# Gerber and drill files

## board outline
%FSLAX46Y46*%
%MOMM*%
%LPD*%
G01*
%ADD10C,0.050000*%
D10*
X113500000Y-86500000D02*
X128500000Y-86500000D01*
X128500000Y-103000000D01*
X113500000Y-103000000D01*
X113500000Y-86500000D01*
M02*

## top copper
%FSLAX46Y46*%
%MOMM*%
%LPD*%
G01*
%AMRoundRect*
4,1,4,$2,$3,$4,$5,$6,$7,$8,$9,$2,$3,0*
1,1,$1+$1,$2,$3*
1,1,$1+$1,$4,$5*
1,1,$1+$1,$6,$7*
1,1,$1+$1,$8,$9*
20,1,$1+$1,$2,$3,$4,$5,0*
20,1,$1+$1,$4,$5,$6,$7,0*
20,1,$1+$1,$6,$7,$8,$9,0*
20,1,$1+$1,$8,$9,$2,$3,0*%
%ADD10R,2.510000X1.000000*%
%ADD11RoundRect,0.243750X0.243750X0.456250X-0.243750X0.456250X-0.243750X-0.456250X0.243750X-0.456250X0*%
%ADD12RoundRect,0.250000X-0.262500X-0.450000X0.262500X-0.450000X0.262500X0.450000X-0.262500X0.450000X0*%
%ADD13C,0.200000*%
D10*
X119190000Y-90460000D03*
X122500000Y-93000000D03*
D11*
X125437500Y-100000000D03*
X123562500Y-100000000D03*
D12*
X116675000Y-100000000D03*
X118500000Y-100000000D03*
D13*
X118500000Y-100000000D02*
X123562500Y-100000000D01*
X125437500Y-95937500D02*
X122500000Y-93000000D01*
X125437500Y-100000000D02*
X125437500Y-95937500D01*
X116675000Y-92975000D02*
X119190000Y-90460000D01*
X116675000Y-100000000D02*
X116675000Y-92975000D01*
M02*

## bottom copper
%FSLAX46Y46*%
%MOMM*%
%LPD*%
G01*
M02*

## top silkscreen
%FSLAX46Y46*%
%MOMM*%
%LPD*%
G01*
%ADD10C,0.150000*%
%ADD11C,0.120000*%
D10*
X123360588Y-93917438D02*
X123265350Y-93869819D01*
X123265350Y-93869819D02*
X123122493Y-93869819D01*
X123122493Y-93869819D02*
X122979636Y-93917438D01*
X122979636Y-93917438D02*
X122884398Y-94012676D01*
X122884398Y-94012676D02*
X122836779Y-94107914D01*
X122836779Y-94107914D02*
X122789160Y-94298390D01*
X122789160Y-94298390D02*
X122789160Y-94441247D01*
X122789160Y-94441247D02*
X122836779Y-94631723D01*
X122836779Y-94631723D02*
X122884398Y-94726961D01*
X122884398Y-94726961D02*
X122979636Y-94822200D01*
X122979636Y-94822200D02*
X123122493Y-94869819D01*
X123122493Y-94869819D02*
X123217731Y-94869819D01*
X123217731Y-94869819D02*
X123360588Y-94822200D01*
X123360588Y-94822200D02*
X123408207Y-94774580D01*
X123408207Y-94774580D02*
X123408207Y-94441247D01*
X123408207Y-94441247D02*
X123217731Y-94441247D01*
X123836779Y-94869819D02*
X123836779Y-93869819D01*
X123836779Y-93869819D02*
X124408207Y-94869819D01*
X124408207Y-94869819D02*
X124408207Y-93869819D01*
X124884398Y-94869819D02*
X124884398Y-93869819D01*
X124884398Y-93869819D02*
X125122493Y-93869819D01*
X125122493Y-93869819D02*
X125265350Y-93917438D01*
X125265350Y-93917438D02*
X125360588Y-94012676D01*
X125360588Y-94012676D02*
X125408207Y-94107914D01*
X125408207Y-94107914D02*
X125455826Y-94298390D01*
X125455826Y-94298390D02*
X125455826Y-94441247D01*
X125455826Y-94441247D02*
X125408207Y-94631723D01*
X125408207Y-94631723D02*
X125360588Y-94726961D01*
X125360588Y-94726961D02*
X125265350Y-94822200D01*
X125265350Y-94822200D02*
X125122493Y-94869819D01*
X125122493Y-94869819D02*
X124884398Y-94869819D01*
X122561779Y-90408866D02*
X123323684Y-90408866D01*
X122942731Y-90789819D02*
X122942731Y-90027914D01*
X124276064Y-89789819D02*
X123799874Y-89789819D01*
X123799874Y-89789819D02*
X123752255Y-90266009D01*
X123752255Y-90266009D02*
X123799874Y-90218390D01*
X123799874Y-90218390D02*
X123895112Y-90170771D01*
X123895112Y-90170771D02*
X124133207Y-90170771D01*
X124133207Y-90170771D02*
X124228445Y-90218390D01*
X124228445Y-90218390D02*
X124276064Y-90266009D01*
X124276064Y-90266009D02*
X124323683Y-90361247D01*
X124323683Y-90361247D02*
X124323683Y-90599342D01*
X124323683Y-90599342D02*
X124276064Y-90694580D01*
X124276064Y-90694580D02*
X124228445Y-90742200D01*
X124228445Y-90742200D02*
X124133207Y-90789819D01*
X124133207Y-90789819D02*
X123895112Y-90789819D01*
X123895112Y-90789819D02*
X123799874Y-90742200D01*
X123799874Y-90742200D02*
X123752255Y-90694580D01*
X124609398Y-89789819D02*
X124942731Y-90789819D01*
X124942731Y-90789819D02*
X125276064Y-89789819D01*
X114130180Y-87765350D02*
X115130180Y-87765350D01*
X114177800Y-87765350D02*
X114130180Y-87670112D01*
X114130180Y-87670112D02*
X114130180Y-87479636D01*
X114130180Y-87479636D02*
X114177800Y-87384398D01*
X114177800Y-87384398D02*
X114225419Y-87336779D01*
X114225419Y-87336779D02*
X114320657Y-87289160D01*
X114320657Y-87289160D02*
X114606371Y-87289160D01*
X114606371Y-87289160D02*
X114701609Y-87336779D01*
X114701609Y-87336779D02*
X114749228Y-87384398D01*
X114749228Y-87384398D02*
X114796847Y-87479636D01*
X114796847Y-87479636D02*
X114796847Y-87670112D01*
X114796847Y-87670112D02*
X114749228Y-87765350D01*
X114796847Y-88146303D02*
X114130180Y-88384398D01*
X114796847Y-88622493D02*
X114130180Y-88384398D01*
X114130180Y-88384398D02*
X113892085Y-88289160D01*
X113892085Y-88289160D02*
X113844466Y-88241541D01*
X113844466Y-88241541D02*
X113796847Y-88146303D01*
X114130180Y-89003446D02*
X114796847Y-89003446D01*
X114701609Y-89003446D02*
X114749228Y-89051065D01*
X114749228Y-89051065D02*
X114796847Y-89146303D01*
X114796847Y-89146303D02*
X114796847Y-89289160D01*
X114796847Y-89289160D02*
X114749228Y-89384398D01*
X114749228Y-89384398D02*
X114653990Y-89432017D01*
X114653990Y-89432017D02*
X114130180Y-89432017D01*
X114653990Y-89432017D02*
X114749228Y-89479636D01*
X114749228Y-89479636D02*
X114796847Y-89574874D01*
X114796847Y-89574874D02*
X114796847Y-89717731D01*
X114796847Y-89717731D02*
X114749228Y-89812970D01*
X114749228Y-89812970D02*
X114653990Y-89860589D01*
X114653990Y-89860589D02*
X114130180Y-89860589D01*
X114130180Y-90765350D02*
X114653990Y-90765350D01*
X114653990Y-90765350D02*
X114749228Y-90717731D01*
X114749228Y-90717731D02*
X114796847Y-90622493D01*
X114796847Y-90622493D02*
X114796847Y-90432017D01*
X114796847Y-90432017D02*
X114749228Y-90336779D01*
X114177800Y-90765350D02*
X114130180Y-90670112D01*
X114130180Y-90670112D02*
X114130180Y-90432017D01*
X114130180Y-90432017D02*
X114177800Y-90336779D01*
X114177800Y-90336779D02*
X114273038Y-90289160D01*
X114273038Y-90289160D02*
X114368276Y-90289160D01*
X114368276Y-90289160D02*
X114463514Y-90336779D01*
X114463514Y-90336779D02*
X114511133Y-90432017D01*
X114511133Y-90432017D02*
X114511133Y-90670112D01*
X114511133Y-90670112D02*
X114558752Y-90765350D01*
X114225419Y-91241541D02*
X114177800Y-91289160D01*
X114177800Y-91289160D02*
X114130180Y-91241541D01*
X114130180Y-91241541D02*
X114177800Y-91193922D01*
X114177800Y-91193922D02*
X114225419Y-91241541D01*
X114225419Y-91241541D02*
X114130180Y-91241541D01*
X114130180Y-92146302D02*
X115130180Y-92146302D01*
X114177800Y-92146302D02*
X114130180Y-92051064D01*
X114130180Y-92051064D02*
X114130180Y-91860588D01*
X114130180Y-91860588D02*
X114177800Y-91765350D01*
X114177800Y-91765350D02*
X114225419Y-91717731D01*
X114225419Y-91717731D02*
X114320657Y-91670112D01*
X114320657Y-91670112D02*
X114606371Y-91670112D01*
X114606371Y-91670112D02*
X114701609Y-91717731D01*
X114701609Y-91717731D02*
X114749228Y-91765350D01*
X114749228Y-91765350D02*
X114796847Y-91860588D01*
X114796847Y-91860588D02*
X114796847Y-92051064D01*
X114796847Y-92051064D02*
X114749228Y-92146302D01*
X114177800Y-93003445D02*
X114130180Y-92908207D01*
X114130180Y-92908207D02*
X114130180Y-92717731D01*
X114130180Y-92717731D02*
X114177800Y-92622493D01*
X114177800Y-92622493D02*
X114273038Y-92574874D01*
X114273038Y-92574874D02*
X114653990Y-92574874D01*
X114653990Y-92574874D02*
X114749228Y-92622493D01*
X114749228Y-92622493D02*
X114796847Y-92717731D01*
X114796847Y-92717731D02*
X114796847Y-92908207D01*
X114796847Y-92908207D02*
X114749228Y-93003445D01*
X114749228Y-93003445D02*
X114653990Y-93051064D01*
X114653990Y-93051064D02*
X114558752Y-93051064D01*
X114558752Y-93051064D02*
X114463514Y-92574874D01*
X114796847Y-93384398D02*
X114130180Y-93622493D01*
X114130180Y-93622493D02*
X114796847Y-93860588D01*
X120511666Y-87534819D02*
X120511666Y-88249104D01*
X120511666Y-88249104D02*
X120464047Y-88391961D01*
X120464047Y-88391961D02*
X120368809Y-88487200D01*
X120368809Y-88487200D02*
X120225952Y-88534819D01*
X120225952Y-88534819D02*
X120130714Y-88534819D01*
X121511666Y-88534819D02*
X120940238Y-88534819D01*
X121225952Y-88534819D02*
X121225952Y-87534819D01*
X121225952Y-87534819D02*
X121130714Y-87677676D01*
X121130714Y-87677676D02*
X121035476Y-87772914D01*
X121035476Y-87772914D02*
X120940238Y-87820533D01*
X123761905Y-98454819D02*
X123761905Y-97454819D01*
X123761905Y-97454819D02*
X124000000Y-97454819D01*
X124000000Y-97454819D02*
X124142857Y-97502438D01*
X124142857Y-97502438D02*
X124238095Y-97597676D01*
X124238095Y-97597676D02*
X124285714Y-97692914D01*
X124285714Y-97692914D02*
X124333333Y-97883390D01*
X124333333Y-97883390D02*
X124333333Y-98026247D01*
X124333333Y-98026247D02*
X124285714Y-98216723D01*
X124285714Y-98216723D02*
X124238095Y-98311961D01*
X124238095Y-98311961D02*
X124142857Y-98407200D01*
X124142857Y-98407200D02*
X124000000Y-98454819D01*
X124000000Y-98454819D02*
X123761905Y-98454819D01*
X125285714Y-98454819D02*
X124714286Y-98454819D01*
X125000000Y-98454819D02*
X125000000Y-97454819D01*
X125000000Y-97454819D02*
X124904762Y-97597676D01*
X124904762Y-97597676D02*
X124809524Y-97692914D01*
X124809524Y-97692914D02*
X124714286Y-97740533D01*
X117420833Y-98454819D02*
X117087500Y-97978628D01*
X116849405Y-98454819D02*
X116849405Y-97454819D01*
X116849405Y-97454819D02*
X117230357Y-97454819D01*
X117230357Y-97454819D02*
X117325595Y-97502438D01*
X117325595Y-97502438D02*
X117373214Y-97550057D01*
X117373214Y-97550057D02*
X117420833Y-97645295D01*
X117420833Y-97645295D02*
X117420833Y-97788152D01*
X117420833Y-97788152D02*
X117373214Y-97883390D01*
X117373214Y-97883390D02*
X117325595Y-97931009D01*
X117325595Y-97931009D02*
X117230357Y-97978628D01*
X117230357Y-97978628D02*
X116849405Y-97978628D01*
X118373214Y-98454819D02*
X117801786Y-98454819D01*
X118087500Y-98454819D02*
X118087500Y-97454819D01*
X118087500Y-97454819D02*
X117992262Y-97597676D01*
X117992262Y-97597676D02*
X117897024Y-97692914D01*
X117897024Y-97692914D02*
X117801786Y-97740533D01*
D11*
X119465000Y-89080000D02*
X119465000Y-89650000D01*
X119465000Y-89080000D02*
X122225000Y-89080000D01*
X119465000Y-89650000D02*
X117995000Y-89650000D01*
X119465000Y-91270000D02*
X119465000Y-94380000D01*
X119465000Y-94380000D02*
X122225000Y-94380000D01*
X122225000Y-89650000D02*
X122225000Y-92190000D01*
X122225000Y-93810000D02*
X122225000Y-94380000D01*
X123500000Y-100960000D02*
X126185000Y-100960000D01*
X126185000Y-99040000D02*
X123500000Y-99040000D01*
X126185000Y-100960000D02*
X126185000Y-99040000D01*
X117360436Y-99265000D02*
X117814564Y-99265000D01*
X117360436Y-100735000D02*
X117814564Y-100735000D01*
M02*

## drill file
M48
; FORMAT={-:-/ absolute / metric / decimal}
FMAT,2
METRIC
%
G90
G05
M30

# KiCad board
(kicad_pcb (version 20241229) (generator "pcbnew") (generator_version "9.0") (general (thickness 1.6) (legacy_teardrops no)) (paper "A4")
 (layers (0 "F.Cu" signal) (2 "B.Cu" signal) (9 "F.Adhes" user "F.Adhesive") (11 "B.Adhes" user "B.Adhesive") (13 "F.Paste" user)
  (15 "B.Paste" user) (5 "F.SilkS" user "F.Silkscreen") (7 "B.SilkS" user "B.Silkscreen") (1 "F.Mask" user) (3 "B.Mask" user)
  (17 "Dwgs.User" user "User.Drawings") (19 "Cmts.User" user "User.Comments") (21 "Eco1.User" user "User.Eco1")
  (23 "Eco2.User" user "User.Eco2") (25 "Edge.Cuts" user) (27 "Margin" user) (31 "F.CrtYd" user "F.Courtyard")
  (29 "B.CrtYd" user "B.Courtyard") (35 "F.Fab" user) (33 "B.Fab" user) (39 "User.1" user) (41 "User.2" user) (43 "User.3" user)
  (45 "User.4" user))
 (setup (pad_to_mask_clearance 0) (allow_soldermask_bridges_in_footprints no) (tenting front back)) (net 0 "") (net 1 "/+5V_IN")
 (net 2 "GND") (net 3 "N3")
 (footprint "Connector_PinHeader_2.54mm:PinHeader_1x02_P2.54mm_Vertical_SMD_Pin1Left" (layer "F.Cu") (at 120.845 91.73)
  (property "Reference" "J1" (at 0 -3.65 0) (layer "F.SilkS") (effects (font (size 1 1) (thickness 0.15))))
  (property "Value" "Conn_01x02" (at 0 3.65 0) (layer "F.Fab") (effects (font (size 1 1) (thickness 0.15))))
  (fp_line (start -1.38 -2.65) (end -1.38 -2.08) (stroke (width 0.12) (type solid)) (layer "F.SilkS"))
  (fp_line (start -1.38 -2.65) (end 1.38 -2.65) (stroke (width 0.12) (type solid)) (layer "F.SilkS"))
  (fp_line (start -1.38 -2.08) (end -2.85 -2.08) (stroke (width 0.12) (type solid)) (layer "F.SilkS"))
  (fp_line (start -1.38 -0.46) (end -1.38 2.65) (stroke (width 0.12) (type solid)) (layer "F.SilkS"))
  (fp_line (start -1.38 2.65) (end 1.38 2.65) (stroke (width 0.12) (type solid)) (layer "F.SilkS"))
  (fp_line (start 1.38 -2.08) (end 1.38 0.46) (stroke (width 0.12) (type solid)) (layer "F.SilkS"))
  (fp_line (start 1.38 2.08) (end 1.38 2.65) (stroke (width 0.12) (type solid)) (layer "F.SilkS"))
  (pad "1" smd rect (at -1.655 -1.27) (size 2.51 1) (layers "F.Cu" "F.Mask" "F.Paste") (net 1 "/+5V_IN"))
  (pad "2" smd rect (at 1.655 1.27) (size 2.51 1) (layers "F.Cu" "F.Mask" "F.Paste") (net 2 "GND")))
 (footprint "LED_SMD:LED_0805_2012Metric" (layer "F.Cu") (at 124.5 100 180)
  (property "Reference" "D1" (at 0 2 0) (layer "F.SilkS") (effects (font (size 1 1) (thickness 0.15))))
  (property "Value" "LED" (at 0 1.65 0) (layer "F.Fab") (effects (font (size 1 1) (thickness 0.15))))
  (fp_line (start 1 -0.96) (end -1.685 -0.96) (stroke (width 0.12) (type solid)) (layer "F.SilkS"))
  (fp_line (start -1.685 0.96) (end 1 0.96) (stroke (width 0.12) (type solid)) (layer "F.SilkS"))
  (fp_line (start -1.685 -0.96) (end -1.685 0.96) (stroke (width 0.12) (type solid)) (layer "F.SilkS"))
  (pad "1" smd roundrect (at -0.9375 0 180) (size 0.975 1.4) (layers "F.Cu" "F.Mask" "F.Paste") (roundrect_rratio 0.25) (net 2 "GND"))
  (pad "2" smd roundrect (at 0.9375 0 180) (size 0.975 1.4) (layers "F.Cu" "F.Mask" "F.Paste") (roundrect_rratio 0.25) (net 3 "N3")))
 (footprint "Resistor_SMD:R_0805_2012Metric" (layer "F.Cu") (at 117.5875 100)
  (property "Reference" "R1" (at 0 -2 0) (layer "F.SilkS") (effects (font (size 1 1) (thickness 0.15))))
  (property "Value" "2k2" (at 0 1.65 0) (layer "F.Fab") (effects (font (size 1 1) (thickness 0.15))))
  (fp_line (start -0.227064 -0.735) (end 0.227064 -0.735) (stroke (width 0.12) (type solid)) (layer "F.SilkS"))
  (fp_line (start -0.227064 0.735) (end 0.227064 0.735) (stroke (width 0.12) (type solid)) (layer "F.SilkS"))
  (pad "1" smd roundrect (at -0.9125 0) (size 1.025 1.4) (layers "F.Cu" "F.Mask" "F.Paste") (roundrect_rratio 0.243902) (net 1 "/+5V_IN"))
  (pad "2" smd roundrect (at 0.9125 0) (size 1.025 1.4) (layers "F.Cu" "F.Mask" "F.Paste") (roundrect_rratio 0.243902) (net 3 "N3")))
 (gr_rect (start 113.5 86.5) (end 128.5 103) (stroke (width 0.05) (type default)) (fill no) (layer "Edge.Cuts"))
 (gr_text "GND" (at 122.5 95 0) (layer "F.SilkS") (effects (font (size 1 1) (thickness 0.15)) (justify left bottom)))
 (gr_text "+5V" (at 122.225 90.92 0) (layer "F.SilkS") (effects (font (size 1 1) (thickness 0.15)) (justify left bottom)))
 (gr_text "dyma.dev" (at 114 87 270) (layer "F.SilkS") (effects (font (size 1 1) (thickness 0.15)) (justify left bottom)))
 (segment (start 118.5 100) (end 123.5625 100) (width 0.2) (layer "F.Cu") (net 3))
 (segment (start 125.4375 95.9375) (end 122.5 93) (width 0.2) (layer "F.Cu") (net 2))
 (segment (start 125.4375 100) (end 125.4375 95.9375) (width 0.2) (layer "F.Cu") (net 2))
 (segment (start 116.675 92.975) (end 119.19 90.46) (width 0.2) (layer "F.Cu") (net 1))
 (segment (start 116.675 100) (end 116.675 92.975) (width 0.2) (layer "F.Cu") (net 1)))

